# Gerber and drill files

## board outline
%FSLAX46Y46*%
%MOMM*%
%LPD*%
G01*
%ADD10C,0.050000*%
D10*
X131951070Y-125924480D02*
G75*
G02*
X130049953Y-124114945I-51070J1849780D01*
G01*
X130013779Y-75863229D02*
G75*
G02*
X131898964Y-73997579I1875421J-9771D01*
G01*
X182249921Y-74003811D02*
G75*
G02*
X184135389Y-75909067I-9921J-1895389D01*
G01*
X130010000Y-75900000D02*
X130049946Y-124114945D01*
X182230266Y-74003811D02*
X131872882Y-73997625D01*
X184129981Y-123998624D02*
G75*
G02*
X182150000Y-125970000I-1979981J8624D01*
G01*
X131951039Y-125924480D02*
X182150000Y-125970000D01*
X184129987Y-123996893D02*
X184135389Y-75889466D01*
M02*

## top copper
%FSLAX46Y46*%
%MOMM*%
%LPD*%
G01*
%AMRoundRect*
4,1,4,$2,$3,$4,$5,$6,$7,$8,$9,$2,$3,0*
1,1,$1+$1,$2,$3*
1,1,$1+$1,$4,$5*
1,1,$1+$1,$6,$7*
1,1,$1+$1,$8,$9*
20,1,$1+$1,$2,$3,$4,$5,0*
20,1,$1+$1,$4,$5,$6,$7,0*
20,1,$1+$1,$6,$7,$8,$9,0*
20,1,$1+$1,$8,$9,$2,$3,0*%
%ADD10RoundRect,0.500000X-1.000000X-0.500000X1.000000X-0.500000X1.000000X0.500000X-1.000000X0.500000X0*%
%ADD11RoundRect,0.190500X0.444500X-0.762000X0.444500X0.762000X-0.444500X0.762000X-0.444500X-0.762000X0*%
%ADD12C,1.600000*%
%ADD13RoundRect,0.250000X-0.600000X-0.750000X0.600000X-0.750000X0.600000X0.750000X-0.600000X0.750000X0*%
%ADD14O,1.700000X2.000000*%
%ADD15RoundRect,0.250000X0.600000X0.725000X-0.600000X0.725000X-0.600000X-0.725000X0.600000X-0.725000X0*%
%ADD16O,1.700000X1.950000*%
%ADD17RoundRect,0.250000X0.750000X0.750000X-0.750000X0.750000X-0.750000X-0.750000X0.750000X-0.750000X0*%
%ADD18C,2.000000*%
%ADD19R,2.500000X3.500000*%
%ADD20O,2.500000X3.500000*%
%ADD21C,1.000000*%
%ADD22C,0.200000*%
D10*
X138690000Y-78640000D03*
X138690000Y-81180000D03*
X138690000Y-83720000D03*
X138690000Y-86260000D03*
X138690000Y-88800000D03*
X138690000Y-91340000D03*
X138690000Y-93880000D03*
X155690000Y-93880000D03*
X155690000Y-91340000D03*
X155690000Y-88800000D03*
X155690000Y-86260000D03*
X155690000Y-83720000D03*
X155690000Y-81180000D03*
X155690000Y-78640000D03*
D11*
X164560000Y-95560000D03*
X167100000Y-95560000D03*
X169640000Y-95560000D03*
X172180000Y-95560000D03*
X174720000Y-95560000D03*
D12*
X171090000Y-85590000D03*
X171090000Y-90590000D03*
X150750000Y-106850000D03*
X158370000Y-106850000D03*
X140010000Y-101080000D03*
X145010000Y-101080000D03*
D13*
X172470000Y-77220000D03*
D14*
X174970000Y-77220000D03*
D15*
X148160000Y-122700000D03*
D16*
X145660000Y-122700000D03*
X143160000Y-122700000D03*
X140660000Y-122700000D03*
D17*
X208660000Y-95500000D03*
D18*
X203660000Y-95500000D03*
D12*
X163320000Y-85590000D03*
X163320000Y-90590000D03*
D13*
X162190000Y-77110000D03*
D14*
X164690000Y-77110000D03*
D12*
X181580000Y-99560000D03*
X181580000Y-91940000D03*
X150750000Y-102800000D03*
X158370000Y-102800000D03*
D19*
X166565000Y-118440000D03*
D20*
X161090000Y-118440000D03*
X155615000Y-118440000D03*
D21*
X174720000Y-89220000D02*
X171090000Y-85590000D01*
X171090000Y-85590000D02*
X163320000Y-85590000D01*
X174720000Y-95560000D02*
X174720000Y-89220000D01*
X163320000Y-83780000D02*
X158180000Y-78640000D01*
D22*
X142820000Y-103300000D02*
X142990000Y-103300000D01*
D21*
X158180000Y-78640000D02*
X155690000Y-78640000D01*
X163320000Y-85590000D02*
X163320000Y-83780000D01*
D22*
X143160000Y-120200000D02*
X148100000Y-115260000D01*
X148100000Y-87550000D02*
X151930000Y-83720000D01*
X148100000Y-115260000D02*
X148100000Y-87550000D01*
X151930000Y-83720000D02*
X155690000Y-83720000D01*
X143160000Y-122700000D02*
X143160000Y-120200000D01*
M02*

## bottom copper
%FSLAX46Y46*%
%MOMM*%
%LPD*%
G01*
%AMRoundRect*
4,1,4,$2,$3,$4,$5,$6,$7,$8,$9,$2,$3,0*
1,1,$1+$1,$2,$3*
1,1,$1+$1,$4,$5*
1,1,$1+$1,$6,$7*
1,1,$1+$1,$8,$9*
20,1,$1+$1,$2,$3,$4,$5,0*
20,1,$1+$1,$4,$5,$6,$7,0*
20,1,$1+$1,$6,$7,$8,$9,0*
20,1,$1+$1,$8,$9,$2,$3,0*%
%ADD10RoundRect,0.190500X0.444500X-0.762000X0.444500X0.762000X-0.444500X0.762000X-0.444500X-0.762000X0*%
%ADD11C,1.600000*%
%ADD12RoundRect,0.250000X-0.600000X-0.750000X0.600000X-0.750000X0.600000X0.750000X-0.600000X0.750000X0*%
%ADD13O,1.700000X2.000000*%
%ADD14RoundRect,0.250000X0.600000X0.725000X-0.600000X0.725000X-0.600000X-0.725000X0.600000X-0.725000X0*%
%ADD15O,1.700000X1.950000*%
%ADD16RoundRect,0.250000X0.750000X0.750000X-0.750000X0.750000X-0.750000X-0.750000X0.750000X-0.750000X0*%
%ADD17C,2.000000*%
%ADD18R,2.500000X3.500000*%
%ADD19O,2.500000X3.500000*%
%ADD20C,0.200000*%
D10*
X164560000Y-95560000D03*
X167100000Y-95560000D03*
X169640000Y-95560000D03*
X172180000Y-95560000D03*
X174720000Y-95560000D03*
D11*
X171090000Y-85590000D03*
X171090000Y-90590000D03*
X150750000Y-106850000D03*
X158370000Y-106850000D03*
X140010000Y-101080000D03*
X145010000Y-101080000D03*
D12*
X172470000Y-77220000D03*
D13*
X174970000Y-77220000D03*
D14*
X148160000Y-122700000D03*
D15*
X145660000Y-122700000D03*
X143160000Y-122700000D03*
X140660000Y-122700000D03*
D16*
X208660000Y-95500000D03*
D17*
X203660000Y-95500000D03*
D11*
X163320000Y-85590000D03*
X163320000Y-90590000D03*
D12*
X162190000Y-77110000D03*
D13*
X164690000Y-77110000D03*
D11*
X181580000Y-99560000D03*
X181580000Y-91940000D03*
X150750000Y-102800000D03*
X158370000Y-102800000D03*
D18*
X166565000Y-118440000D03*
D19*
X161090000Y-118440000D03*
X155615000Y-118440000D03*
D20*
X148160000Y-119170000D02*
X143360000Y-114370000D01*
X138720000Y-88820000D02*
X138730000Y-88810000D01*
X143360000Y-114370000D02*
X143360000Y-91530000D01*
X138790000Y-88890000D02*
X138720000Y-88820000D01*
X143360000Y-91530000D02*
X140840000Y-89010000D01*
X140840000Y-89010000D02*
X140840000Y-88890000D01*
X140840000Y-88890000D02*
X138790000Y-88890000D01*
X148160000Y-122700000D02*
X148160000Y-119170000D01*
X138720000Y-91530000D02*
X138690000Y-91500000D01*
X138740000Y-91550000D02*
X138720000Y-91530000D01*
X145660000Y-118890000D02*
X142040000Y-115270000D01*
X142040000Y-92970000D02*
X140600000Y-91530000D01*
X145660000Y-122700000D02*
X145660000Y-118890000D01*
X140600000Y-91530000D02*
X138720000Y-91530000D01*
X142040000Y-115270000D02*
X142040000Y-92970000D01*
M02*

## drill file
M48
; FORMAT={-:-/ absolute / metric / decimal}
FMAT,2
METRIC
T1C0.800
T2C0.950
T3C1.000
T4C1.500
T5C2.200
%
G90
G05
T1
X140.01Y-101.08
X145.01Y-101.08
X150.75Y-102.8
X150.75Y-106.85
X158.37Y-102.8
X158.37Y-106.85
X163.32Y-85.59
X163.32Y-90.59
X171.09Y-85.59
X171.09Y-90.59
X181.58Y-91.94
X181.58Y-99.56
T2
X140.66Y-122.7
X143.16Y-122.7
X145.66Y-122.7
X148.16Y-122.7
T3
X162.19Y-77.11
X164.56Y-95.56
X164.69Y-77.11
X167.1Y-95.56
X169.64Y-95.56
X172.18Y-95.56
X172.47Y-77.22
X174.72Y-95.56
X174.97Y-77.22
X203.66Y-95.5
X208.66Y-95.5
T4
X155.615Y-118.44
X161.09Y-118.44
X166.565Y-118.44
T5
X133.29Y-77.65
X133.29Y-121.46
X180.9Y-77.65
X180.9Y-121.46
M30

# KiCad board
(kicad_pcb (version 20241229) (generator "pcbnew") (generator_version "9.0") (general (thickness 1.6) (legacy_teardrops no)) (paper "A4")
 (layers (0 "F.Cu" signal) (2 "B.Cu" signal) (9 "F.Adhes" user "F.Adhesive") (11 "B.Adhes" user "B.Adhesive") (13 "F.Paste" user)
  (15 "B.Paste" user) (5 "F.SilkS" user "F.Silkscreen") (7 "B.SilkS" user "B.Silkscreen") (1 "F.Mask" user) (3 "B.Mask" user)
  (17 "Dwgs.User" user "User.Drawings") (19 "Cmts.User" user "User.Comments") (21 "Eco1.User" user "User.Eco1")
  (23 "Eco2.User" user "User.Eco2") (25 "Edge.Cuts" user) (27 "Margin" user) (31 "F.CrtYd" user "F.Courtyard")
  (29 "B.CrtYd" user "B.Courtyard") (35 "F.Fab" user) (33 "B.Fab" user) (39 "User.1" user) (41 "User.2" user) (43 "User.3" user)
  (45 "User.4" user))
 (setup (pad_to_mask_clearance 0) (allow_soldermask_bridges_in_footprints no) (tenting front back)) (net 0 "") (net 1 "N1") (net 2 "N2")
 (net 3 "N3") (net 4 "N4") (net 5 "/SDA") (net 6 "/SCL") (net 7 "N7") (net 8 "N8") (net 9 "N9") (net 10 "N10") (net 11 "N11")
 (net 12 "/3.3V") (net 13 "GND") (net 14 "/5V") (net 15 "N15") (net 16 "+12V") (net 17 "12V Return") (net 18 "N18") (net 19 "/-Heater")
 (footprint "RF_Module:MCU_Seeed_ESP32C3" (layer "F.Cu") (at 147.19 86.26)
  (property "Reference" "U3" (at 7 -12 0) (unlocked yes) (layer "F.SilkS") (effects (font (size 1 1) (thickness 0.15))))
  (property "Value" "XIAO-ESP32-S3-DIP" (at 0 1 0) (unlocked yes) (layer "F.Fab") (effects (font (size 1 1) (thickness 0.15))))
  (pad "1" smd roundrect (at -8.5 -7.62) (size 3 2) (layers "F.Cu" "F.Mask" "F.Paste") (roundrect_rratio 0.25) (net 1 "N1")
   (thermal_bridge_angle 45))
  (pad "2" smd roundrect (at -8.5 -5.08) (size 3 2) (layers "F.Cu" "F.Mask" "F.Paste") (roundrect_rratio 0.25) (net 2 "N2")
   (thermal_bridge_angle 45))
  (pad "3" smd roundrect (at -8.5 -2.54) (size 3 2) (layers "F.Cu" "F.Mask" "F.Paste") (roundrect_rratio 0.25) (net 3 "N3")
   (thermal_bridge_angle 45))
  (pad "4" smd roundrect (at -8.5 0) (size 3 2) (layers "F.Cu" "F.Mask" "F.Paste") (roundrect_rratio 0.25) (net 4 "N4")
   (thermal_bridge_angle 45))
  (pad "5" smd roundrect (at -8.5 2.54) (size 3 2) (layers "F.Cu" "F.Mask" "F.Paste") (roundrect_rratio 0.25) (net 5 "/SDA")
   (thermal_bridge_angle 45))
  (pad "6" smd roundrect (at -8.5 5.08) (size 3 2) (layers "F.Cu" "F.Mask" "F.Paste") (roundrect_rratio 0.25) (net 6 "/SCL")
   (thermal_bridge_angle 45))
  (pad "7" smd roundrect (at -8.5 7.62) (size 3 2) (layers "F.Cu" "F.Mask" "F.Paste") (roundrect_rratio 0.25) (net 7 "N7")
   (thermal_bridge_angle 45))
  (pad "8" smd roundrect (at 8.5 7.62) (size 3 2) (layers "F.Cu" "F.Mask" "F.Paste") (roundrect_rratio 0.25) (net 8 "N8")
   (thermal_bridge_angle 45))
  (pad "9" smd roundrect (at 8.5 5.08) (size 3 2) (layers "F.Cu" "F.Mask" "F.Paste") (roundrect_rratio 0.25) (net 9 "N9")
   (thermal_bridge_angle 45))
  (pad "10" smd roundrect (at 8.5 2.54) (size 3 2) (layers "F.Cu" "F.Mask" "F.Paste") (roundrect_rratio 0.25) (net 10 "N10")
   (thermal_bridge_angle 45))
  (pad "11" smd roundrect (at 8.5 0) (size 3 2) (layers "F.Cu" "F.Mask" "F.Paste") (roundrect_rratio 0.25) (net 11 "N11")
   (thermal_bridge_angle 45))
  (pad "12" smd roundrect (at 8.5 -2.54) (size 3 2) (layers "F.Cu" "F.Mask" "F.Paste") (roundrect_rratio 0.25) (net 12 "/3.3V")
   (thermal_bridge_angle 45))
  (pad "13" smd roundrect (at 8.5 -5.08) (size 3 2) (layers "F.Cu" "F.Mask" "F.Paste") (roundrect_rratio 0.25) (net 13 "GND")
   (thermal_bridge_angle 45))
  (pad "14" smd roundrect (at 8.5 -7.62) (size 3 2) (layers "F.Cu" "F.Mask" "F.Paste") (roundrect_rratio 0.25) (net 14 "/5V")
   (thermal_bridge_angle 45)))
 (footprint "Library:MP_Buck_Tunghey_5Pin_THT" (layer "F.Cu") (at 169.64 103.56 90)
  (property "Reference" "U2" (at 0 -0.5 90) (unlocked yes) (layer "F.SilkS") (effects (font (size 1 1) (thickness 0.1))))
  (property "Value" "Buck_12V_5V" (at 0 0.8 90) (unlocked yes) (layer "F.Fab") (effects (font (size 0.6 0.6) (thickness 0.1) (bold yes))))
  (pad "1" thru_hole roundrect (at 8 -5.08 90) (size 1.905 1.27) (drill 1) (layers "*.Cu" "*.Mask") (remove_unused_layers no)
   (roundrect_rratio 0.15) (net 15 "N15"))
  (pad "2" thru_hole roundrect (at 8 -2.54 90) (size 1.905 1.27) (drill 1) (layers "*.Cu" "*.Mask") (remove_unused_layers no)
   (roundrect_rratio 0.15) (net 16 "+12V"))
  (pad "3" thru_hole roundrect (at 8 0 90) (size 1.905 1.27) (drill 1) (layers "*.Cu" "*.Mask") (remove_unused_layers no)
   (roundrect_rratio 0.15) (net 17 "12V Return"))
  (pad "4" thru_hole roundrect (at 8 2.54 90) (size 1.905 1.27) (drill 1) (layers "*.Cu" "*.Mask") (remove_unused_layers no)
   (roundrect_rratio 0.15) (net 13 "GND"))
  (pad "5" thru_hole roundrect (at 8 5.08 90) (size 1.905 1.27) (drill 1) (layers "*.Cu" "*.Mask") (remove_unused_layers no)
   (roundrect_rratio 0.15) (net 14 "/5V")))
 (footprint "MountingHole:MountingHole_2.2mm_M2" (layer "F.Cu") (at 133.29 121.46)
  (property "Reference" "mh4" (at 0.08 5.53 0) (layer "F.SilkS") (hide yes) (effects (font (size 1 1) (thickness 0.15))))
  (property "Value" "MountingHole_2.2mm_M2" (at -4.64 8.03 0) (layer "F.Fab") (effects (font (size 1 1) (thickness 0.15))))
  (pad "" np_thru_hole circle (at 0 0) (size 2.2 2.2) (drill 2.2) (layers "*.Cu" "*.Mask")))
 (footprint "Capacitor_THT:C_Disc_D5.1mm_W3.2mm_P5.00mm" (layer "F.Cu") (at 171.09 85.59 -90)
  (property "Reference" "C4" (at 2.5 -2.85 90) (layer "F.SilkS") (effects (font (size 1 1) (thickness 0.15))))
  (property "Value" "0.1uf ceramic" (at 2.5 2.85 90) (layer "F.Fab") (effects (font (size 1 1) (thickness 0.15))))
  (pad "1" thru_hole circle (at 0 0 270) (size 1.6 1.6) (drill 0.8) (layers "*.Cu" "*.Mask") (remove_unused_layers no) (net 14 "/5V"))
  (pad "2" thru_hole circle (at 5 0 270) (size 1.6 1.6) (drill 0.8) (layers "*.Cu" "*.Mask") (remove_unused_layers no) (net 13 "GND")))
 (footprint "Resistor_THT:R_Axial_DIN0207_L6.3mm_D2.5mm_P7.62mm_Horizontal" (layer "F.Cu") (at 150.75 106.85)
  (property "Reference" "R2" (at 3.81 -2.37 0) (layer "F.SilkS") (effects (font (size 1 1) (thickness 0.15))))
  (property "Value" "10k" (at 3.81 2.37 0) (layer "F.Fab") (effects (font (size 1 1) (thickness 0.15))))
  (pad "1" thru_hole circle (at 0 0) (size 1.6 1.6) (drill 0.8) (layers "*.Cu" "*.Mask") (remove_unused_layers no) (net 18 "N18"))
  (pad "2" thru_hole circle (at 7.62 0) (size 1.6 1.6) (drill 0.8) (layers "*.Cu" "*.Mask") (remove_unused_layers no) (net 13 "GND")))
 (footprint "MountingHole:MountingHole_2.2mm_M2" (layer "F.Cu") (at 180.9 121.46)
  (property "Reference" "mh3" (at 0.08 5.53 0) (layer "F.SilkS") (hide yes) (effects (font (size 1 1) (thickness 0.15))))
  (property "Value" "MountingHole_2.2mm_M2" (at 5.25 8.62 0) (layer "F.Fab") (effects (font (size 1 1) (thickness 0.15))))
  (pad "" np_thru_hole circle (at 0 0) (size 2.2 2.2) (drill 2.2) (layers "*.Cu" "*.Mask")))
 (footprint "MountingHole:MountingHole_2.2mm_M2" (layer "F.Cu") (at 180.9 77.65)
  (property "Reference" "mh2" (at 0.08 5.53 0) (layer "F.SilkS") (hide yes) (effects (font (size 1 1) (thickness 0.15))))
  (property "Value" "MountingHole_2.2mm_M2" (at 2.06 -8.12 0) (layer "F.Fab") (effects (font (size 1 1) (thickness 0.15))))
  (pad "" np_thru_hole circle (at 0 0) (size 2.2 2.2) (drill 2.2) (layers "*.Cu" "*.Mask")))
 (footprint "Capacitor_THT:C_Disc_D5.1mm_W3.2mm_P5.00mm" (layer "F.Cu") (at 140.01 101.08)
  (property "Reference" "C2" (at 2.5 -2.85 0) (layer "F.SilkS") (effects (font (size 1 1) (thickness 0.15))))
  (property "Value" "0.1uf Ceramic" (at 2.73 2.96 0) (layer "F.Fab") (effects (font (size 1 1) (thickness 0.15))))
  (pad "1" thru_hole circle (at 0 0) (size 1.6 1.6) (drill 0.8) (layers "*.Cu" "*.Mask") (remove_unused_layers no) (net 16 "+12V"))
  (pad "2" thru_hole circle (at 5 0) (size 1.6 1.6) (drill 0.8) (layers "*.Cu" "*.Mask") (remove_unused_layers no) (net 17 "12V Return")))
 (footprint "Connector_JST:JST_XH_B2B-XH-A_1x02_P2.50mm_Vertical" (layer "F.Cu") (at 172.47 77.22)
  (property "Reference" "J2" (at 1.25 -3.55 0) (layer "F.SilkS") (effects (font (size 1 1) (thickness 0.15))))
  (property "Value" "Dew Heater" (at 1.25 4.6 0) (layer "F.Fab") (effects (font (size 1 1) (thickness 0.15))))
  (pad "1" thru_hole roundrect (at 0 0) (size 1.7 2) (drill 1) (layers "*.Cu" "*.Mask") (remove_unused_layers no)
   (roundrect_rratio 0.147059) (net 16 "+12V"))
  (pad "2" thru_hole oval (at 2.5 0) (size 1.7 2) (drill 1) (layers "*.Cu" "*.Mask") (remove_unused_layers no) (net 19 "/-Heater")))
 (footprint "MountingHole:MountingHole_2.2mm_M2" (layer "F.Cu") (at 133.29 77.65)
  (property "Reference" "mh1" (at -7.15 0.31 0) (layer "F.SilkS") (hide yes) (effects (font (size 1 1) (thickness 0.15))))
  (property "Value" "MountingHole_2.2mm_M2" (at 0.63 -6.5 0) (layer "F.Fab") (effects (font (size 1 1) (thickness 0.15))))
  (pad "" np_thru_hole circle (at 0 0) (size 2.2 2.2) (drill 2.2) (layers "*.Cu" "*.Mask")))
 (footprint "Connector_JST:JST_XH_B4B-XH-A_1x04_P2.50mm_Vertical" (layer "F.Cu") (at 148.16 122.7 180)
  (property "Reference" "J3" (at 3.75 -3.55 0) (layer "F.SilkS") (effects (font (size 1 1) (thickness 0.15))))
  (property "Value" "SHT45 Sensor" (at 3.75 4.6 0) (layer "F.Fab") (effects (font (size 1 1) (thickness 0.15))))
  (pad "1" thru_hole roundrect (at 0 0 180) (size 1.7 1.95) (drill 0.95) (layers "*.Cu" "*.Mask") (remove_unused_layers no)
   (roundrect_rratio 0.147059) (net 5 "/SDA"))
  (pad "2" thru_hole oval (at 2.5 0 180) (size 1.7 1.95) (drill 0.95) (layers "*.Cu" "*.Mask") (remove_unused_layers no) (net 6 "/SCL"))
  (pad "3" thru_hole oval (at 5 0 180) (size 1.7 1.95) (drill 0.95) (layers "*.Cu" "*.Mask") (remove_unused_layers no) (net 12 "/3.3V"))
  (pad "4" thru_hole oval (at 7.5 0 180) (size 1.7 1.95) (drill 0.95) (layers "*.Cu" "*.Mask") (remove_unused_layers no) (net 13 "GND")))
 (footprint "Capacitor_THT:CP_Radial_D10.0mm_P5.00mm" (layer "F.Cu") (at 208.66 95.5 180)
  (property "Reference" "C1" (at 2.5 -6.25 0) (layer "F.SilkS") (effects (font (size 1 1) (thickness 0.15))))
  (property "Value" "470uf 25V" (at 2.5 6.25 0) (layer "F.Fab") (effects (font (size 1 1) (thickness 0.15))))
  (pad "1" thru_hole roundrect (at 0 0 180) (size 2 2) (drill 1) (layers "*.Cu" "*.Mask") (remove_unused_layers no) (roundrect_rratio 0.125)
   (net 16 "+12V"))
  (pad "2" thru_hole circle (at 5 0 180) (size 2 2) (drill 1) (layers "*.Cu" "*.Mask") (remove_unused_layers no) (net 17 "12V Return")))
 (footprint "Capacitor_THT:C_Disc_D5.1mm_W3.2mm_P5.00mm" (layer "F.Cu") (at 163.32 85.59 -90)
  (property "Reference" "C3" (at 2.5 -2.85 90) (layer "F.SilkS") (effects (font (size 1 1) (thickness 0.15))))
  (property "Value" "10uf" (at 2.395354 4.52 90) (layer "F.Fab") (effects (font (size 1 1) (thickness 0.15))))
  (pad "1" thru_hole circle (at 0 0 270) (size 1.6 1.6) (drill 0.8) (layers "*.Cu" "*.Mask") (remove_unused_layers no) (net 14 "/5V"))
  (pad "2" thru_hole circle (at 5 0 270) (size 1.6 1.6) (drill 0.8) (layers "*.Cu" "*.Mask") (remove_unused_layers no) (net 13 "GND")))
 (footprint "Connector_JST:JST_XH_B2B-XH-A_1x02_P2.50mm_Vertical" (layer "F.Cu") (at 162.19 77.11)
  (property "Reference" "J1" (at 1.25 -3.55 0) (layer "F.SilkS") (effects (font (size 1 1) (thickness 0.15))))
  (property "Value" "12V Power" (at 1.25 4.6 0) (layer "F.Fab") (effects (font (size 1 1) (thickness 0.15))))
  (pad "1" thru_hole roundrect (at 0 0) (size 1.7 2) (drill 1) (layers "*.Cu" "*.Mask") (remove_unused_layers no)
   (roundrect_rratio 0.147059) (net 16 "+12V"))
  (pad "2" thru_hole oval (at 2.5 0) (size 1.7 2) (drill 1) (layers "*.Cu" "*.Mask") (remove_unused_layers no) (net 17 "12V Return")))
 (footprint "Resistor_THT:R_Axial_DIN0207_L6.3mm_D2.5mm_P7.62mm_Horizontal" (layer "F.Cu") (at 181.58 99.56 90)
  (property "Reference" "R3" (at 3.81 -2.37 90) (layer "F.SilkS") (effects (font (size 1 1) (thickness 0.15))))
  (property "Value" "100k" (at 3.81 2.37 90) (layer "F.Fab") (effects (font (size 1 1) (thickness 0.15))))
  (pad "1" thru_hole circle (at 0 0 90) (size 1.6 1.6) (drill 0.8) (layers "*.Cu" "*.Mask") (remove_unused_layers no) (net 16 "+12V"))
  (pad "2" thru_hole circle (at 7.62 0 90) (size 1.6 1.6) (drill 0.8) (layers "*.Cu" "*.Mask") (remove_unused_layers no) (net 15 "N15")))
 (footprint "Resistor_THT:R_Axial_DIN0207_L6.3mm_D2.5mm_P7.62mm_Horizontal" (layer "F.Cu") (at 150.75 102.8)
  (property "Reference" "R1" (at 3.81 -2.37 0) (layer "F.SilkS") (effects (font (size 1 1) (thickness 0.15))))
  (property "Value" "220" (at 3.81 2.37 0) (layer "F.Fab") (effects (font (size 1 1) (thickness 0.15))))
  (pad "1" thru_hole circle (at 0 0) (size 1.6 1.6) (drill 0.8) (layers "*.Cu" "*.Mask") (remove_unused_layers no) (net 9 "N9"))
  (pad "2" thru_hole circle (at 7.62 0) (size 1.6 1.6) (drill 0.8) (layers "*.Cu" "*.Mask") (remove_unused_layers no) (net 18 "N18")))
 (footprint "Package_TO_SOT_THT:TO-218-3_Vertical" (layer "F.Cu") (at 166.565 118.44 180)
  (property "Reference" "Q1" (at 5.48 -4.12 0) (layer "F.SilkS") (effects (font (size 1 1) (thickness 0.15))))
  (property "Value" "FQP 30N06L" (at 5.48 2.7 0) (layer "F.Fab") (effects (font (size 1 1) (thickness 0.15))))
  (pad "1" thru_hole rect (at 0 0 180) (size 2.5 3.5) (drill 1.5) (layers "*.Cu" "*.Mask") (remove_unused_layers no) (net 18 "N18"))
  (pad "2" thru_hole oval (at 5.475 0 180) (size 2.5 3.5) (drill 1.5) (layers "*.Cu" "*.Mask") (remove_unused_layers no) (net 19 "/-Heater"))
  (pad "3" thru_hole oval (at 10.95 0 180) (size 2.5 3.5) (drill 1.5) (layers "*.Cu" "*.Mask") (remove_unused_layers no) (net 13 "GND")))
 (gr_arc (start 131.95107 125.92448) (mid 130.62419 125.415077) (end 130.049946 124.114945) (stroke (width 0.05) (type default))
  (layer "Edge.Cuts"))
 (gr_arc (start 130.013779 75.863229) (mid 130.57 74.54) (end 131.898964 73.997625) (stroke (width 0.05) (type default)) (layer "Edge.Cuts"))
 (gr_arc (start 182.249921 74.003811) (mid 183.587239 74.565954) (end 184.135389 75.909067) (stroke (width 0.05) (type default))
  (layer "Edge.Cuts"))
 (gr_line (start 130.01 75.9) (end 130.049946 124.114945) (stroke (width 0.05) (type default)) (layer "Edge.Cuts"))
 (gr_line (start 182.230266 74.003811) (end 131.872882 73.997625) (stroke (width 0.05) (type default)) (layer "Edge.Cuts"))
 (gr_arc (start 184.129981 123.998624) (mid 183.547019 125.393117) (end 182.15 125.97) (stroke (width 0.05) (type default))
  (layer "Edge.Cuts"))
 (gr_line (start 131.951039 125.92448) (end 182.15 125.97) (stroke (width 0.05) (type default)) (layer "Edge.Cuts"))
 (gr_line (start 184.129987 123.996893) (end 184.135389 75.889466) (stroke (width 0.05) (type default)) (layer "Edge.Cuts"))
 (segment (start 174.72 89.22) (end 171.09 85.59) (width 1) (layer "F.Cu") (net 14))
 (segment (start 171.09 85.59) (end 163.32 85.59) (width 1) (layer "F.Cu") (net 14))
 (segment (start 174.72 95.56) (end 174.72 89.22) (width 1) (layer "F.Cu") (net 14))
 (segment (start 163.32 83.78) (end 158.18 78.64) (width 1) (layer "F.Cu") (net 14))
 (segment (start 142.82 103.3) (end 142.99 103.3) (width 0.2) (layer "F.Cu") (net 14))
 (segment (start 158.18 78.64) (end 155.69 78.64) (width 1) (layer "F.Cu") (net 14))
 (segment (start 163.32 85.59) (end 163.32 83.78) (width 1) (layer "F.Cu") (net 14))
 (segment (start 143.16 120.2) (end 148.1 115.26) (width 0.2) (layer "F.Cu") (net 12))
 (segment (start 148.1 87.55) (end 151.93 83.72) (width 0.2) (layer "F.Cu") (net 12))
 (segment (start 148.1 115.26) (end 148.1 87.55) (width 0.2) (layer "F.Cu") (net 12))
 (segment (start 151.93 83.72) (end 155.69 83.72) (width 0.2) (layer "F.Cu") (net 12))
 (segment (start 143.16 122.7) (end 143.16 120.2) (width 0.2) (layer "F.Cu") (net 12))
 (segment (start 148.16 119.17) (end 143.36 114.37) (width 0.2) (layer "B.Cu") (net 5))
 (segment (start 138.72 88.82) (end 138.73 88.81) (width 0.2) (layer "B.Cu") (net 5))
 (segment (start 143.36 114.37) (end 143.36 91.53) (width 0.2) (layer "B.Cu") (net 5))
 (segment (start 138.79 88.89) (end 138.72 88.82) (width 0.2) (layer "B.Cu") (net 5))
 (segment (start 143.36 91.53) (end 140.84 89.01) (width 0.2) (layer "B.Cu") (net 5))
 (segment (start 140.84 89.01) (end 140.84 88.89) (width 0.2) (layer "B.Cu") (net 5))
 (segment (start 140.84 88.89) (end 138.79 88.89) (width 0.2) (layer "B.Cu") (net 5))
 (segment (start 148.16 122.7) (end 148.16 119.17) (width 0.2) (layer "B.Cu") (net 5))
 (segment (start 138.72 91.53) (end 138.69 91.5) (width 0.2) (layer "B.Cu") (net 6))
 (segment (start 138.74 91.55) (end 138.72 91.53) (width 0.2) (layer "B.Cu") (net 6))
 (segment (start 145.66 118.89) (end 142.04 115.27) (width 0.2) (layer "B.Cu") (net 6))
 (segment (start 142.04 92.97) (end 140.6 91.53) (width 0.2) (layer "B.Cu") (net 6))
 (segment (start 145.66 122.7) (end 145.66 118.89) (width 0.2) (layer "B.Cu") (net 6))
 (segment (start 140.6 91.53) (end 138.72 91.53) (width 0.2) (layer "B.Cu") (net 6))
 (segment (start 142.04 115.27) (end 142.04 92.97) (width 0.2) (layer "B.Cu") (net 6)))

